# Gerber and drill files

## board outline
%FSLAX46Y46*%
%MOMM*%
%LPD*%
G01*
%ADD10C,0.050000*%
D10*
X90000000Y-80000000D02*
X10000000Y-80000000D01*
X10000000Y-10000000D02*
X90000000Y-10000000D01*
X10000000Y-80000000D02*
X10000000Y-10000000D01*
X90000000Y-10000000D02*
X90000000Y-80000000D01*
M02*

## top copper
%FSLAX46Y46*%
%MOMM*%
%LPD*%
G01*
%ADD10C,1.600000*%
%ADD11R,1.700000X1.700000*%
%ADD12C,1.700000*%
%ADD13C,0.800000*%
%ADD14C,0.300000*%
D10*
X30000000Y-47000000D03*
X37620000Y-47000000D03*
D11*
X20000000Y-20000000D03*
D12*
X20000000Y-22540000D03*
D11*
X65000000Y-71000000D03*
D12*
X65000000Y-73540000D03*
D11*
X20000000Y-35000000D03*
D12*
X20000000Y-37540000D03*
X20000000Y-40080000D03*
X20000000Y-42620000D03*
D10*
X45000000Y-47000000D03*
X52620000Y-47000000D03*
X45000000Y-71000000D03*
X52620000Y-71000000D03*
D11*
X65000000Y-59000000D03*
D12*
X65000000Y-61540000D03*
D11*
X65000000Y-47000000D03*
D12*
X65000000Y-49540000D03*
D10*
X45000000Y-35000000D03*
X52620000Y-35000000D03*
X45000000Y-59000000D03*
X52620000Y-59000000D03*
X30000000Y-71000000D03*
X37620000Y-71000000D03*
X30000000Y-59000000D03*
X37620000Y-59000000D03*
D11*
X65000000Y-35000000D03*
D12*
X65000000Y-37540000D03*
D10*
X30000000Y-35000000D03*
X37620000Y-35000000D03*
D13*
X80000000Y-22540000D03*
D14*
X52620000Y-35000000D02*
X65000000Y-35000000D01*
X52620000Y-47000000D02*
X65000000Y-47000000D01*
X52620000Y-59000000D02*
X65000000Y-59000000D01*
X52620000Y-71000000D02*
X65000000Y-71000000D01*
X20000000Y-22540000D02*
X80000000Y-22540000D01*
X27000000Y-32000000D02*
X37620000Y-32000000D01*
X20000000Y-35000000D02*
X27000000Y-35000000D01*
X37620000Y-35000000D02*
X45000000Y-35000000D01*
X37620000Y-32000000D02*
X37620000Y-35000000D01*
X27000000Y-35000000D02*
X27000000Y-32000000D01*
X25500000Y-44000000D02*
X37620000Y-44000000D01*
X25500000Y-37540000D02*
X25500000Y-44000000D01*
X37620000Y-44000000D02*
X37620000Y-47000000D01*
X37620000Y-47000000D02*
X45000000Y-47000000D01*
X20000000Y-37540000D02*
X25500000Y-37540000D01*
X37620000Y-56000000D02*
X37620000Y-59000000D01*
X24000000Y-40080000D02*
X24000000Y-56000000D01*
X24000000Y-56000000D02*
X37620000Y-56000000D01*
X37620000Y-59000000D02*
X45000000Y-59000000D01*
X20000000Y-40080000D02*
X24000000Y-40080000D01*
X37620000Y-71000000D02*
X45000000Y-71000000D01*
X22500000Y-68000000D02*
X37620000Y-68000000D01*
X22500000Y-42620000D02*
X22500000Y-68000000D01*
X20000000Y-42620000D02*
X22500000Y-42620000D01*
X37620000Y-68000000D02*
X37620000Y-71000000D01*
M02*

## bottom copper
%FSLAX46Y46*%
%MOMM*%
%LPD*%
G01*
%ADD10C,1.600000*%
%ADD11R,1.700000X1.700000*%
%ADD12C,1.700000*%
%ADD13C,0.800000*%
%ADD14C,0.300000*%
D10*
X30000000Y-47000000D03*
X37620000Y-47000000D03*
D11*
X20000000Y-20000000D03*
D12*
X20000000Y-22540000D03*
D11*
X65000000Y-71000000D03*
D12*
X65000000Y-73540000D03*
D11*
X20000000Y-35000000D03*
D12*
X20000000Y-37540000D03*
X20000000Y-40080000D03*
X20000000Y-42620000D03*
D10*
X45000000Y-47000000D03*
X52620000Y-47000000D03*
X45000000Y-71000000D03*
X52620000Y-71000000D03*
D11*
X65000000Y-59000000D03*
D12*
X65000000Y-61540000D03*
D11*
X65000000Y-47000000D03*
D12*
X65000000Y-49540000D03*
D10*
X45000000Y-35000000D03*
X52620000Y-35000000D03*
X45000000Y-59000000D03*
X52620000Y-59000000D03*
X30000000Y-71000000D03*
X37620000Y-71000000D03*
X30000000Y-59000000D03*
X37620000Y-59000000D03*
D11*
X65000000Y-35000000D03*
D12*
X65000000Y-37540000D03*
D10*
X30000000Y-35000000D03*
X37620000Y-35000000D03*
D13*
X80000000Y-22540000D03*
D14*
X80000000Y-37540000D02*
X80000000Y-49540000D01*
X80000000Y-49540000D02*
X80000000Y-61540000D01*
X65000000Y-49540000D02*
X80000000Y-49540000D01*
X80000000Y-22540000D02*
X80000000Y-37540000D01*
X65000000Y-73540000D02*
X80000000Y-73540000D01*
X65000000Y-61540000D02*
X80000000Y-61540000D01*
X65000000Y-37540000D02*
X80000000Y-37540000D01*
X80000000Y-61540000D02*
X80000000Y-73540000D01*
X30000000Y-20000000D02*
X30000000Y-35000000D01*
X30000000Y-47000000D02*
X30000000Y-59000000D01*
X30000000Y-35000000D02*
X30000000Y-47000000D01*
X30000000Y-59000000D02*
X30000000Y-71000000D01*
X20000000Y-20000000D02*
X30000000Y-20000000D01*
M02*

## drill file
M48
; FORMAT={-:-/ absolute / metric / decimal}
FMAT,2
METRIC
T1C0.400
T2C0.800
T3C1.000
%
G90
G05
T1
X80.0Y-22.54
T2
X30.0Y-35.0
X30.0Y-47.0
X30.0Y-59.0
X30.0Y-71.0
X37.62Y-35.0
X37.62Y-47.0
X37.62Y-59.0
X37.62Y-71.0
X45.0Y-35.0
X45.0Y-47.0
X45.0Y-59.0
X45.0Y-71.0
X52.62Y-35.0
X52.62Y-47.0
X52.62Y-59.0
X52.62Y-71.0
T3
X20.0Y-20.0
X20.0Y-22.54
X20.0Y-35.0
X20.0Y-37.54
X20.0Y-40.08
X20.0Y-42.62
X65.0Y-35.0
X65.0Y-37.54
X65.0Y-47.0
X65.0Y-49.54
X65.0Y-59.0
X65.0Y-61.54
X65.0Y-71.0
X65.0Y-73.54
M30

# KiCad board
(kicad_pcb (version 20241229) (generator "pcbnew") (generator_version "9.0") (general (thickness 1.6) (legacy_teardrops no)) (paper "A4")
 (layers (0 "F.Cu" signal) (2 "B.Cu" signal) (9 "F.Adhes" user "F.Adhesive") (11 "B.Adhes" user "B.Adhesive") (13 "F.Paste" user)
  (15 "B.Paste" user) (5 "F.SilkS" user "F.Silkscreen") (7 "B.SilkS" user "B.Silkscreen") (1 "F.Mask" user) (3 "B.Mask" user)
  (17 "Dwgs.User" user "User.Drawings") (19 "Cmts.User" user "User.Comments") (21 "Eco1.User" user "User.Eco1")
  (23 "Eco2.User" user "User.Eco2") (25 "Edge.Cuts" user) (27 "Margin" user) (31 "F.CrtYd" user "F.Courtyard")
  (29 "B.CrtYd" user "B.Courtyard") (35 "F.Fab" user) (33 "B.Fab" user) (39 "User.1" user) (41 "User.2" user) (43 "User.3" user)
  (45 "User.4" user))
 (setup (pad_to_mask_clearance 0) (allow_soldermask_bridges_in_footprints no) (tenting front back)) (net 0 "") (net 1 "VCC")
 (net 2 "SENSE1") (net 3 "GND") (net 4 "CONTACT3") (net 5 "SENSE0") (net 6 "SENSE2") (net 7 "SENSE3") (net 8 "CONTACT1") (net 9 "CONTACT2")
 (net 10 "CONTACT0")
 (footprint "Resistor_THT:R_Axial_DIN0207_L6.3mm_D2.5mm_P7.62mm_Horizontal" (layer "F.Cu") (at 30 47)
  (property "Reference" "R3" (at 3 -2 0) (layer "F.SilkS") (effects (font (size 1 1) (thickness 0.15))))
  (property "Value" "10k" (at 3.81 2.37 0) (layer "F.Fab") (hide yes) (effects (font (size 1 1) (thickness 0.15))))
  (pad "1" thru_hole circle (at 0 0) (size 1.6 1.6) (drill 0.8) (layers "*.Cu" "*.Mask") (remove_unused_layers no) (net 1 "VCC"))
  (pad "2" thru_hole circle (at 7.62 0) (size 1.6 1.6) (drill 0.8) (layers "*.Cu" "*.Mask") (remove_unused_layers no) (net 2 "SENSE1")))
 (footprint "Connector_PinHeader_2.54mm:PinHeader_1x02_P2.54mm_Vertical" (layer "F.Cu") (at 20 20)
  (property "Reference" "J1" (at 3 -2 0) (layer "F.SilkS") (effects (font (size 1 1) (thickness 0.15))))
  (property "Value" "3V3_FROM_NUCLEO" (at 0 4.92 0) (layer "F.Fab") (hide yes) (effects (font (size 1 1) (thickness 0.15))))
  (pad "1" thru_hole rect (at 0 0) (size 1.7 1.7) (drill 1) (layers "*.Cu" "*.Mask") (remove_unused_layers no) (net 1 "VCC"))
  (pad "2" thru_hole circle (at 0 2.54) (size 1.7 1.7) (drill 1) (layers "*.Cu" "*.Mask") (remove_unused_layers no) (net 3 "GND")))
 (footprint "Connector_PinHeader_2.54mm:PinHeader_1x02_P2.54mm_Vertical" (layer "F.Cu") (at 65 71)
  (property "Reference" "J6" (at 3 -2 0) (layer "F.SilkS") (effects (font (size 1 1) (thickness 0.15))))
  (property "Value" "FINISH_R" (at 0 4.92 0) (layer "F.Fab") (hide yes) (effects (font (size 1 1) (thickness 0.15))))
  (pad "1" thru_hole rect (at 0 0) (size 1.7 1.7) (drill 1) (layers "*.Cu" "*.Mask") (remove_unused_layers no) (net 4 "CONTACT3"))
  (pad "2" thru_hole circle (at 0 2.54) (size 1.7 1.7) (drill 1) (layers "*.Cu" "*.Mask") (remove_unused_layers no) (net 3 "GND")))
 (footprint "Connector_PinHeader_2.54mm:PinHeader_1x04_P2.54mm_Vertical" (layer "F.Cu") (at 20 35)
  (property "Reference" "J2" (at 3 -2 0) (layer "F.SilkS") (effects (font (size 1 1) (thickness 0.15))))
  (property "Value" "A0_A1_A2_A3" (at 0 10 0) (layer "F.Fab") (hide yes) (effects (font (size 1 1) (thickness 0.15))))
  (pad "1" thru_hole rect (at 0 0) (size 1.7 1.7) (drill 1) (layers "*.Cu" "*.Mask") (remove_unused_layers no) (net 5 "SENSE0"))
  (pad "2" thru_hole circle (at 0 2.54) (size 1.7 1.7) (drill 1) (layers "*.Cu" "*.Mask") (remove_unused_layers no) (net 2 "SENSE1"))
  (pad "3" thru_hole circle (at 0 5.08) (size 1.7 1.7) (drill 1) (layers "*.Cu" "*.Mask") (remove_unused_layers no) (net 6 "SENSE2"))
  (pad "4" thru_hole circle (at 0 7.62) (size 1.7 1.7) (drill 1) (layers "*.Cu" "*.Mask") (remove_unused_layers no) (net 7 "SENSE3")))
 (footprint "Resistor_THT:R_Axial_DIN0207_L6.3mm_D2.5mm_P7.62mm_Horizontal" (layer "F.Cu") (at 45 47)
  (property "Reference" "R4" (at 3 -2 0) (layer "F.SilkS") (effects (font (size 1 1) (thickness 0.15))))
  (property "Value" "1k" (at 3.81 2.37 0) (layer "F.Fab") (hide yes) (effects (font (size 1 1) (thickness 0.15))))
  (pad "1" thru_hole circle (at 0 0) (size 1.6 1.6) (drill 0.8) (layers "*.Cu" "*.Mask") (remove_unused_layers no) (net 2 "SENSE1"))
  (pad "2" thru_hole circle (at 7.62 0) (size 1.6 1.6) (drill 0.8) (layers "*.Cu" "*.Mask") (remove_unused_layers no) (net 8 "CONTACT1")))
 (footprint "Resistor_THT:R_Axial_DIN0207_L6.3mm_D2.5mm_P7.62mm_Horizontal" (layer "F.Cu") (at 45 71)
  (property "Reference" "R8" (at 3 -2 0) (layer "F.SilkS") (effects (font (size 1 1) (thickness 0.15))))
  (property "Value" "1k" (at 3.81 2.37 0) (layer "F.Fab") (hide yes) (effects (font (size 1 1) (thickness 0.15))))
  (pad "1" thru_hole circle (at 0 0) (size 1.6 1.6) (drill 0.8) (layers "*.Cu" "*.Mask") (remove_unused_layers no) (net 7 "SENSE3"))
  (pad "2" thru_hole circle (at 7.62 0) (size 1.6 1.6) (drill 0.8) (layers "*.Cu" "*.Mask") (remove_unused_layers no) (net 4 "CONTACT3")))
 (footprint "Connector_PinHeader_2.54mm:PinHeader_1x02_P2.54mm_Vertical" (layer "F.Cu") (at 65 59)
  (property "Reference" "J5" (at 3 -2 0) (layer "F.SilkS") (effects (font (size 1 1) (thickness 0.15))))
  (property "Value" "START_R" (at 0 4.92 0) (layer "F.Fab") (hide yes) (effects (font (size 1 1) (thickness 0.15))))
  (pad "1" thru_hole rect (at 0 0) (size 1.7 1.7) (drill 1) (layers "*.Cu" "*.Mask") (remove_unused_layers no) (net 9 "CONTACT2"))
  (pad "2" thru_hole circle (at 0 2.54) (size 1.7 1.7) (drill 1) (layers "*.Cu" "*.Mask") (remove_unused_layers no) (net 3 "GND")))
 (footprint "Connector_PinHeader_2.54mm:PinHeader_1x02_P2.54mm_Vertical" (layer "F.Cu") (at 65 47)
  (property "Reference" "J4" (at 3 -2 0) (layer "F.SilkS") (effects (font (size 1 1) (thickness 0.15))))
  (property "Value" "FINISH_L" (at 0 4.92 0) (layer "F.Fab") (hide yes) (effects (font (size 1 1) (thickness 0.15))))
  (pad "1" thru_hole rect (at 0 0) (size 1.7 1.7) (drill 1) (layers "*.Cu" "*.Mask") (remove_unused_layers no) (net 8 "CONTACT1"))
  (pad "2" thru_hole circle (at 0 2.54) (size 1.7 1.7) (drill 1) (layers "*.Cu" "*.Mask") (remove_unused_layers no) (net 3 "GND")))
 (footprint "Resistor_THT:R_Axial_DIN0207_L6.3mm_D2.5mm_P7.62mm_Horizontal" (layer "F.Cu") (at 45 35)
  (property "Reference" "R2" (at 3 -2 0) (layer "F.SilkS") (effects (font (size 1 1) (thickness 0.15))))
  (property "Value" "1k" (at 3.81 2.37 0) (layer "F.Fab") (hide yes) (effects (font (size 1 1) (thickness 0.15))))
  (pad "1" thru_hole circle (at 0 0) (size 1.6 1.6) (drill 0.8) (layers "*.Cu" "*.Mask") (remove_unused_layers no) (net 5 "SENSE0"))
  (pad "2" thru_hole circle (at 7.62 0) (size 1.6 1.6) (drill 0.8) (layers "*.Cu" "*.Mask") (remove_unused_layers no) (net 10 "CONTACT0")))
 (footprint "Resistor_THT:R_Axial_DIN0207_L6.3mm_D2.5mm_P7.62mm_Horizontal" (layer "F.Cu") (at 45 59)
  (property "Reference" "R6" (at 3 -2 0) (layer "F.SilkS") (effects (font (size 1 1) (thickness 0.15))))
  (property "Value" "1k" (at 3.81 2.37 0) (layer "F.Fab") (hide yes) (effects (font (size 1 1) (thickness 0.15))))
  (pad "1" thru_hole circle (at 0 0) (size 1.6 1.6) (drill 0.8) (layers "*.Cu" "*.Mask") (remove_unused_layers no) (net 6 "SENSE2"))
  (pad "2" thru_hole circle (at 7.62 0) (size 1.6 1.6) (drill 0.8) (layers "*.Cu" "*.Mask") (remove_unused_layers no) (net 9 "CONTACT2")))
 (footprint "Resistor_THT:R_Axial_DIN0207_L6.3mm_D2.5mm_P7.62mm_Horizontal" (layer "F.Cu") (at 30 71)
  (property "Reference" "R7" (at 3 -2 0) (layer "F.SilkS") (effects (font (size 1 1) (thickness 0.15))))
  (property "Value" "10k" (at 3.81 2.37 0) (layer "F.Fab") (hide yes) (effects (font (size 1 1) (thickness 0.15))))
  (pad "1" thru_hole circle (at 0 0) (size 1.6 1.6) (drill 0.8) (layers "*.Cu" "*.Mask") (remove_unused_layers no) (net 1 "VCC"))
  (pad "2" thru_hole circle (at 7.62 0) (size 1.6 1.6) (drill 0.8) (layers "*.Cu" "*.Mask") (remove_unused_layers no) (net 7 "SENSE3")))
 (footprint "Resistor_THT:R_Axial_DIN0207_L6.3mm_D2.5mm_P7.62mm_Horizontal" (layer "F.Cu") (at 30 59)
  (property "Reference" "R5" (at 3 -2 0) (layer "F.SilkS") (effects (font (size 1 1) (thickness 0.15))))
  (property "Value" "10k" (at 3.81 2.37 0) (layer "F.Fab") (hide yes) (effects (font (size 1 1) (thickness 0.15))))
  (pad "1" thru_hole circle (at 0 0) (size 1.6 1.6) (drill 0.8) (layers "*.Cu" "*.Mask") (remove_unused_layers no) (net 1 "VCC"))
  (pad "2" thru_hole circle (at 7.62 0) (size 1.6 1.6) (drill 0.8) (layers "*.Cu" "*.Mask") (remove_unused_layers no) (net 6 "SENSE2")))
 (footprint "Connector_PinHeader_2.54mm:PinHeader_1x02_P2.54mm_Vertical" (layer "F.Cu") (at 65 35)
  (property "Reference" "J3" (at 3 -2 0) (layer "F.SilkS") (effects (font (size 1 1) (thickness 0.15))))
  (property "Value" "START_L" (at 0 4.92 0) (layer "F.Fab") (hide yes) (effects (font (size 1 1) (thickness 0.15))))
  (pad "1" thru_hole rect (at 0 0) (size 1.7 1.7) (drill 1) (layers "*.Cu" "*.Mask") (remove_unused_layers no) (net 10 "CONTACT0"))
  (pad "2" thru_hole circle (at 0 2.54) (size 1.7 1.7) (drill 1) (layers "*.Cu" "*.Mask") (remove_unused_layers no) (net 3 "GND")))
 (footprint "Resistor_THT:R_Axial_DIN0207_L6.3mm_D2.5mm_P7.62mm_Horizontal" (layer "F.Cu") (at 30 35)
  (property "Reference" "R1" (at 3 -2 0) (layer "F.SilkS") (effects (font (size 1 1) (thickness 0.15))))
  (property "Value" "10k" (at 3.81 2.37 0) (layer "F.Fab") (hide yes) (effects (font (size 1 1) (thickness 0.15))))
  (pad "1" thru_hole circle (at 0 0) (size 1.6 1.6) (drill 0.8) (layers "*.Cu" "*.Mask") (remove_unused_layers no) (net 1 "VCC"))
  (pad "2" thru_hole circle (at 7.62 0) (size 1.6 1.6) (drill 0.8) (layers "*.Cu" "*.Mask") (remove_unused_layers no) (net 5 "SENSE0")))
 (gr_line (start 90 80) (end 10 80) (stroke (width 0.05) (type default)) (layer "Edge.Cuts"))
 (gr_line (start 10 10) (end 90 10) (stroke (width 0.05) (type default)) (layer "Edge.Cuts"))
 (gr_line (start 10 80) (end 10 10) (stroke (width 0.05) (type default)) (layer "Edge.Cuts"))
 (gr_line (start 90 10) (end 90 80) (stroke (width 0.05) (type default)) (layer "Edge.Cuts"))
 (segment (start 52.62 35) (end 65 35) (width 0.3) (layer "F.Cu") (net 10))
 (segment (start 52.62 47) (end 65 47) (width 0.3) (layer "F.Cu") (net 8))
 (segment (start 52.62 59) (end 65 59) (width 0.3) (layer "F.Cu") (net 9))
 (segment (start 52.62 71) (end 65 71) (width 0.3) (layer "F.Cu") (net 4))
 (segment (start 20 22.54) (end 80 22.54) (width 0.3) (layer "F.Cu") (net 3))
 (via (at 80 22.54) (size 0.8) (drill 0.4) (layers "F.Cu" "B.Cu") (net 3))
 (segment (start 80 37.54) (end 80 49.54) (width 0.3) (layer "B.Cu") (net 3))
 (segment (start 80 49.54) (end 80 61.54) (width 0.3) (layer "B.Cu") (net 3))
 (segment (start 65 49.54) (end 80 49.54) (width 0.3) (layer "B.Cu") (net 3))
 (segment (start 80 22.54) (end 80 37.54) (width 0.3) (layer "B.Cu") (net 3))
 (segment (start 65 73.54) (end 80 73.54) (width 0.3) (layer "B.Cu") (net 3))
 (segment (start 65 61.54) (end 80 61.54) (width 0.3) (layer "B.Cu") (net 3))
 (segment (start 65 37.54) (end 80 37.54) (width 0.3) (layer "B.Cu") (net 3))
 (segment (start 80 61.54) (end 80 73.54) (width 0.3) (layer "B.Cu") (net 3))
 (segment (start 27 32) (end 37.62 32) (width 0.3) (layer "F.Cu") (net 5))
 (segment (start 20 35) (end 27 35) (width 0.3) (layer "F.Cu") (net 5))
 (segment (start 37.62 35) (end 45 35) (width 0.3) (layer "F.Cu") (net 5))
 (segment (start 37.62 32) (end 37.62 35) (width 0.3) (layer "F.Cu") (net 5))
 (segment (start 27 35) (end 27 32) (width 0.3) (layer "F.Cu") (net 5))
 (segment (start 25.5 44) (end 37.62 44) (width 0.3) (layer "F.Cu") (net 2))
 (segment (start 25.5 37.54) (end 25.5 44) (width 0.3) (layer "F.Cu") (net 2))
 (segment (start 37.62 44) (end 37.62 47) (width 0.3) (layer "F.Cu") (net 2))
 (segment (start 37.62 47) (end 45 47) (width 0.3) (layer "F.Cu") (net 2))
 (segment (start 20 37.54) (end 25.5 37.54) (width 0.3) (layer "F.Cu") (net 2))
 (segment (start 37.62 56) (end 37.62 59) (width 0.3) (layer "F.Cu") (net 6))
 (segment (start 24 40.08) (end 24 56) (width 0.3) (layer "F.Cu") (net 6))
 (segment (start 24 56) (end 37.62 56) (width 0.3) (layer "F.Cu") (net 6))
 (segment (start 37.62 59) (end 45 59) (width 0.3) (layer "F.Cu") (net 6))
 (segment (start 20 40.08) (end 24 40.08) (width 0.3) (layer "F.Cu") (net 6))
 (segment (start 37.62 71) (end 45 71) (width 0.3) (layer "F.Cu") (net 7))
 (segment (start 22.5 68) (end 37.62 68) (width 0.3) (layer "F.Cu") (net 7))
 (segment (start 22.5 42.62) (end 22.5 68) (width 0.3) (layer "F.Cu") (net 7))
 (segment (start 20 42.62) (end 22.5 42.62) (width 0.3) (layer "F.Cu") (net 7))
 (segment (start 37.62 68) (end 37.62 71) (width 0.3) (layer "F.Cu") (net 7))
 (segment (start 30 20) (end 30 35) (width 0.3) (layer "B.Cu") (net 1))
 (segment (start 30 47) (end 30 59) (width 0.3) (layer "B.Cu") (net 1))
 (segment (start 30 35) (end 30 47) (width 0.3) (layer "B.Cu") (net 1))
 (segment (start 30 59) (end 30 71) (width 0.3) (layer "B.Cu") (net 1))
 (segment (start 20 20) (end 30 20) (width 0.3) (layer "B.Cu") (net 1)))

